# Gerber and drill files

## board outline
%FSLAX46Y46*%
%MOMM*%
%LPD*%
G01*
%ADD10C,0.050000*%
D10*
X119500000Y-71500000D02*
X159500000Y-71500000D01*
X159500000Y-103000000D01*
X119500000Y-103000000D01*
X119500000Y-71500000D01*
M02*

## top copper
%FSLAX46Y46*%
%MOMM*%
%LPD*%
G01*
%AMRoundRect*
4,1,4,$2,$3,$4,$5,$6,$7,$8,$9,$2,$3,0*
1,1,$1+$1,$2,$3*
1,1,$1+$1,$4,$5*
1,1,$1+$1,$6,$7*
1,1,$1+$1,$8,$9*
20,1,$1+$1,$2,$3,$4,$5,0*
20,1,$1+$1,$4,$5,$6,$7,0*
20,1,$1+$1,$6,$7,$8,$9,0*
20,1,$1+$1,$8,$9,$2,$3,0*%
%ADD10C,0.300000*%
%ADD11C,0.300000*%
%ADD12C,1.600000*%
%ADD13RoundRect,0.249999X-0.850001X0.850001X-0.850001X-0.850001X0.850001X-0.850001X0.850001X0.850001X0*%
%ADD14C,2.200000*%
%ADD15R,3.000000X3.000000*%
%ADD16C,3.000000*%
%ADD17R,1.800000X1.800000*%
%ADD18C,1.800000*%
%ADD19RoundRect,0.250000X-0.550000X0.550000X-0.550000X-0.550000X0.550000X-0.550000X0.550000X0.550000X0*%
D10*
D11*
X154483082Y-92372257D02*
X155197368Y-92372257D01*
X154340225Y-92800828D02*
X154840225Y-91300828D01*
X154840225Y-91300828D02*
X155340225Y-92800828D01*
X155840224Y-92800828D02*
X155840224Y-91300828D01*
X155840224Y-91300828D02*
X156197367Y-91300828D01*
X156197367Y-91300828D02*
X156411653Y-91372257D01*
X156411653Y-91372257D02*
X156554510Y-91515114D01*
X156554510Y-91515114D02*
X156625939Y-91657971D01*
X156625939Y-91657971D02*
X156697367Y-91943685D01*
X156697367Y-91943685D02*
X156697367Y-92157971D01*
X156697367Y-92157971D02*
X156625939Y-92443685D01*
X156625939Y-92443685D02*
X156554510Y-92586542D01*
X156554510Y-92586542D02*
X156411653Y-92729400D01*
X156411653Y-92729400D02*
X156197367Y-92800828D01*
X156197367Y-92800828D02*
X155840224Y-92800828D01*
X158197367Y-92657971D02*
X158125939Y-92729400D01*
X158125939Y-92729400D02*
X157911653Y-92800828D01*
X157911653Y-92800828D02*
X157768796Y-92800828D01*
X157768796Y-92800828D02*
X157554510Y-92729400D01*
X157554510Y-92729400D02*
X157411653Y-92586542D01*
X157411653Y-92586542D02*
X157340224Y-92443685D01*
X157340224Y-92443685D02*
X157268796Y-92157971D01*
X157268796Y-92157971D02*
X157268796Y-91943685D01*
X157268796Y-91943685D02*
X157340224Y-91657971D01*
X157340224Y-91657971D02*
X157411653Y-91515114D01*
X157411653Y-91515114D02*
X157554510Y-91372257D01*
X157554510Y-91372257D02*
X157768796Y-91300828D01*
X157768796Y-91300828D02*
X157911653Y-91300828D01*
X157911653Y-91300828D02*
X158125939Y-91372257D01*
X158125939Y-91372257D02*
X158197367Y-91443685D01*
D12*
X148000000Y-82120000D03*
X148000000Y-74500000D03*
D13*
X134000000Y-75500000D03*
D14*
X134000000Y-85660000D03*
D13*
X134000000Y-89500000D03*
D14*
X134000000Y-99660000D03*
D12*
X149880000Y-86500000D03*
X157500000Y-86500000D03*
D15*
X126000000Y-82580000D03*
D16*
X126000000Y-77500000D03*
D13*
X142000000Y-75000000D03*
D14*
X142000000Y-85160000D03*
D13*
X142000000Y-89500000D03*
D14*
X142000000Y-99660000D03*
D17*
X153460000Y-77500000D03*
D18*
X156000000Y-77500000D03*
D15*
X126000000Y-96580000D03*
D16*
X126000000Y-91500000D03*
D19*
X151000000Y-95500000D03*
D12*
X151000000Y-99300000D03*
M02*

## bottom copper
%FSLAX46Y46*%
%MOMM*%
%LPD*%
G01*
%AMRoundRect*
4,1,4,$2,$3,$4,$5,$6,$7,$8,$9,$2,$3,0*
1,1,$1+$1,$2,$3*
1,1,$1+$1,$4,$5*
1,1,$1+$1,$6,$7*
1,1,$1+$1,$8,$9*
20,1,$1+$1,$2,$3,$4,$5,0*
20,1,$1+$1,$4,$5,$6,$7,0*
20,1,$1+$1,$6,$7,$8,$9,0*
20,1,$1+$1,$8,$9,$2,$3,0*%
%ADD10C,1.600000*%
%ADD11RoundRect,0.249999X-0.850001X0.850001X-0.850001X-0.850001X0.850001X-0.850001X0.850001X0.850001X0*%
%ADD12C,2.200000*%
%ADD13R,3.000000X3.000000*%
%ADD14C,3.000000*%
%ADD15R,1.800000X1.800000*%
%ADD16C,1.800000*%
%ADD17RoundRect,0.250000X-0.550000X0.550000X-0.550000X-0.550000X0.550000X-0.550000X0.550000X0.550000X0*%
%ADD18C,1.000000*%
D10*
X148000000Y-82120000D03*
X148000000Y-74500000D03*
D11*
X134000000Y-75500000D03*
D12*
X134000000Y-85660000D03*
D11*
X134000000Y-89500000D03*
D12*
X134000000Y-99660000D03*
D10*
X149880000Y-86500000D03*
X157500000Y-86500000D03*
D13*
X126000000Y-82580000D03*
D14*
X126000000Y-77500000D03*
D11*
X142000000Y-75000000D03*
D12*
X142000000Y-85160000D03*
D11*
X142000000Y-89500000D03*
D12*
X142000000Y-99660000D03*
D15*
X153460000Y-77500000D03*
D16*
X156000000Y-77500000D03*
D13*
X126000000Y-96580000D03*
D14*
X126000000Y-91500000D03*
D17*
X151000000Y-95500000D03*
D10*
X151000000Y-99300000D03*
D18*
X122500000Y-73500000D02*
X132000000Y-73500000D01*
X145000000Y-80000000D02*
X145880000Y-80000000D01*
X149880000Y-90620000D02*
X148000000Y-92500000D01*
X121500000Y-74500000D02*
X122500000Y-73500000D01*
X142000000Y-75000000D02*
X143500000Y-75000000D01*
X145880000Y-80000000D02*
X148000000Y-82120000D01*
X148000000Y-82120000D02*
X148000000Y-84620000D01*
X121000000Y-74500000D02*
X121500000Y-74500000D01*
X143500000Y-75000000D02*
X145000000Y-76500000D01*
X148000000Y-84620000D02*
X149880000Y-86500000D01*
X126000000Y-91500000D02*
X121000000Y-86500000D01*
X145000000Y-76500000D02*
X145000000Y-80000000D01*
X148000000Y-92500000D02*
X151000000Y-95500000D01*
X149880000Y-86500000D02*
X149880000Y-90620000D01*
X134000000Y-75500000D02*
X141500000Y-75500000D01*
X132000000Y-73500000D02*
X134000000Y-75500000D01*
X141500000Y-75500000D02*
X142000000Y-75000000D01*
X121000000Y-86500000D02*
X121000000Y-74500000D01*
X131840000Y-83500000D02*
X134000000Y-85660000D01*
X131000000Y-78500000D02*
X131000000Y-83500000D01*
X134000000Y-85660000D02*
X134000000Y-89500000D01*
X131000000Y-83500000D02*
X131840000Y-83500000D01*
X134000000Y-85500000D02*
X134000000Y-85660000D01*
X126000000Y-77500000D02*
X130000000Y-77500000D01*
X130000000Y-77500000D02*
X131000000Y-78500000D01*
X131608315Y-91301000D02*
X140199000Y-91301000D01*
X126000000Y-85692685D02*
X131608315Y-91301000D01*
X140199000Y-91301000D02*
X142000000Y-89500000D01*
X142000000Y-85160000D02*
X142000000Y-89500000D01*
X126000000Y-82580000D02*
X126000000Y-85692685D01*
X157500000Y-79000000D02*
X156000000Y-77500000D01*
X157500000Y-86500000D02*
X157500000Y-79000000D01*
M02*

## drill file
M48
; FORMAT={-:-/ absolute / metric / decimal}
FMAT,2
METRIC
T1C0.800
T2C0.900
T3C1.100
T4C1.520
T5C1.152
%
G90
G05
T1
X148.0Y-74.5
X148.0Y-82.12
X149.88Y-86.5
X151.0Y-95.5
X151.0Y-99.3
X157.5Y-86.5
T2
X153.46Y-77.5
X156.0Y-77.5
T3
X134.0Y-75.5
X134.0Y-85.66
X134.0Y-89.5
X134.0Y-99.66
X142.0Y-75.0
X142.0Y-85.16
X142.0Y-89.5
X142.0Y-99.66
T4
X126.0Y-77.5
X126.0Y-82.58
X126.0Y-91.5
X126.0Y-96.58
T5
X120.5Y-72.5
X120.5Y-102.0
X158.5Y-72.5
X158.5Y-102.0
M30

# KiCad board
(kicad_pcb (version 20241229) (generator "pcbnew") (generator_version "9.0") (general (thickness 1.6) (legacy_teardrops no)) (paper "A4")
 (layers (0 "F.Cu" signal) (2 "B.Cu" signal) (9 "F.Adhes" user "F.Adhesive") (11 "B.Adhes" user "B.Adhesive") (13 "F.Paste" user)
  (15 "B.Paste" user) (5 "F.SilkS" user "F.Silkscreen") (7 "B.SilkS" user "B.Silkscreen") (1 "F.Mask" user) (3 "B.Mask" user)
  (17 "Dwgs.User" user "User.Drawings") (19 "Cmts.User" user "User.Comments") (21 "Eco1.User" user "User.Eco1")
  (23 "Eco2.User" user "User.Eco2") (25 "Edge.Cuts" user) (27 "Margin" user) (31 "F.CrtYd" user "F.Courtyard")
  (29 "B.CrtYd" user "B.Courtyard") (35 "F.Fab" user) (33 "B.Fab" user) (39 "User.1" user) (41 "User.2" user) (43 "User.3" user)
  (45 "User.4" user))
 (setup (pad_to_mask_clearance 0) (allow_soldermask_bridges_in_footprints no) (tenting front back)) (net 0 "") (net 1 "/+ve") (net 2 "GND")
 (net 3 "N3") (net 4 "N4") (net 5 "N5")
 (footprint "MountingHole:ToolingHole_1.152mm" (layer "F.Cu") (at 158.5 72.5)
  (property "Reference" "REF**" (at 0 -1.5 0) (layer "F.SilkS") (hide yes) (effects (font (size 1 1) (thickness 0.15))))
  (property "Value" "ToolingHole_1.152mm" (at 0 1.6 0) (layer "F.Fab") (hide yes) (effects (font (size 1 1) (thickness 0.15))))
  (pad "" np_thru_hole circle (at 0 0) (size 1.152 1.152) (drill 1.152) (layers "*.Cu" "*.Mask") (solder_mask_margin 0.074))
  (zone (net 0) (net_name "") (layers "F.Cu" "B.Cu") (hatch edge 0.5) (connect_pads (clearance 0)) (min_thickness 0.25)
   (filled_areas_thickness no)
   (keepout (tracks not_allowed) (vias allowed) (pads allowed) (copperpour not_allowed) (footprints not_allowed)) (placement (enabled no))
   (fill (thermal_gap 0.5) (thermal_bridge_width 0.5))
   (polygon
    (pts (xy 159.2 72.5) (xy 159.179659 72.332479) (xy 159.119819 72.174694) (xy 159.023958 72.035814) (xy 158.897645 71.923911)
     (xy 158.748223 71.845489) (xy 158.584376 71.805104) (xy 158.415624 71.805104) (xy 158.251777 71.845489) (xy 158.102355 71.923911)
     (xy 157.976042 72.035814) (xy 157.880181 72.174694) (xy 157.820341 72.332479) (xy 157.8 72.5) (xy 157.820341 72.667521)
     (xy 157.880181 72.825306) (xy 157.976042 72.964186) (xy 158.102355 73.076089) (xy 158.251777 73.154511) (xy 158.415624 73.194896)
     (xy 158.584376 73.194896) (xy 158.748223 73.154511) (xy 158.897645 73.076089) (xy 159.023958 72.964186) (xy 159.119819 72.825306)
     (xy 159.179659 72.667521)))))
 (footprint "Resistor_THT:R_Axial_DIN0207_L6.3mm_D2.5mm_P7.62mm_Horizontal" (layer "F.Cu") (at 148 82.12 90)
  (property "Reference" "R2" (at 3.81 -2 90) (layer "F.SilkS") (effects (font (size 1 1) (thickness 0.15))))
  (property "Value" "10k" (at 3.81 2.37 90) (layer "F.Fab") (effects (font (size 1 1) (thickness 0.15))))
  (pad "1" thru_hole circle (at 0 0 90) (size 1.6 1.6) (drill 0.8) (layers "*.Cu" "*.Mask") (remove_unused_layers no) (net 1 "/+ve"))
  (pad "2" thru_hole circle (at 7.62 0 90) (size 1.6 1.6) (drill 0.8) (layers "*.Cu" "*.Mask") (remove_unused_layers no) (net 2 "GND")))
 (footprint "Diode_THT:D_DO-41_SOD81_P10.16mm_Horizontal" (layer "F.Cu") (at 134 75.5 -90)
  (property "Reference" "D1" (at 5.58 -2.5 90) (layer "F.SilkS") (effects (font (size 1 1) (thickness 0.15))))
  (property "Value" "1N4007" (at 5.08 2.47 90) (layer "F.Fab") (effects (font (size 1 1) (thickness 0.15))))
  (pad "1" thru_hole roundrect (at 0 0 270) (size 2.2 2.2) (drill 1.1) (layers "*.Cu" "*.Mask") (remove_unused_layers no)
   (roundrect_rratio 0.113636) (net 1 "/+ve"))
  (pad "2" thru_hole circle (at 10.16 0 270) (size 2.2 2.2) (drill 1.1) (layers "*.Cu" "*.Mask") (remove_unused_layers no) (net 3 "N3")))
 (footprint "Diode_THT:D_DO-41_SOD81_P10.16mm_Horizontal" (layer "F.Cu") (at 134 89.5 -90)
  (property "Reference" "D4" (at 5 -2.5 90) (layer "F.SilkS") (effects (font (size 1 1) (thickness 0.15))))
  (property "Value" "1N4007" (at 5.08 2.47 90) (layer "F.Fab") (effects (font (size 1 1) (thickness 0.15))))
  (pad "1" thru_hole roundrect (at 0 0 270) (size 2.2 2.2) (drill 1.1) (layers "*.Cu" "*.Mask") (remove_unused_layers no)
   (roundrect_rratio 0.113636) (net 3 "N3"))
  (pad "2" thru_hole circle (at 10.16 0 270) (size 2.2 2.2) (drill 1.1) (layers "*.Cu" "*.Mask") (remove_unused_layers no) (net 2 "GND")))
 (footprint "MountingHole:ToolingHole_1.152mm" (layer "F.Cu") (at 120.5 72.5)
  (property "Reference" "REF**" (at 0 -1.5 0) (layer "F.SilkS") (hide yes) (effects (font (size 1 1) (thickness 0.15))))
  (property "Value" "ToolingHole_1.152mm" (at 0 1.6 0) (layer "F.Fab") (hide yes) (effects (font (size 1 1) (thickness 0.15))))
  (pad "" np_thru_hole circle (at 0 0) (size 1.152 1.152) (drill 1.152) (layers "*.Cu" "*.Mask") (solder_mask_margin 0.074))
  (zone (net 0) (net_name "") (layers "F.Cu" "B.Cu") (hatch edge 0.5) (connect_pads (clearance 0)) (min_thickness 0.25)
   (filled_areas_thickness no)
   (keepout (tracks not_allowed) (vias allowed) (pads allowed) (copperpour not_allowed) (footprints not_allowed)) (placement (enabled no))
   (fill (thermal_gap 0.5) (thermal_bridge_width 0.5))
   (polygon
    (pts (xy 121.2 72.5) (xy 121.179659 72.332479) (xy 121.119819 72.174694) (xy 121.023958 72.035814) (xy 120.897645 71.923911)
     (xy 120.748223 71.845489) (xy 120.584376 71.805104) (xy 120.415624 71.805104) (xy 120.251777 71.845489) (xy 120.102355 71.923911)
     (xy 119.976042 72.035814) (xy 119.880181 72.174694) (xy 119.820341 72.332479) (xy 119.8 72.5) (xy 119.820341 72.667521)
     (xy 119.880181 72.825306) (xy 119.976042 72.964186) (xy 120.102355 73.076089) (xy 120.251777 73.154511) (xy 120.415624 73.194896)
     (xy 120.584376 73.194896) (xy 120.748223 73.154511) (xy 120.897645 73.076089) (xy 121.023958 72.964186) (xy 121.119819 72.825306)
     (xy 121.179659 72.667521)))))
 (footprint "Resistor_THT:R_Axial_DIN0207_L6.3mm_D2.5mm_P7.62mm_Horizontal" (layer "F.Cu") (at 149.88 86.5)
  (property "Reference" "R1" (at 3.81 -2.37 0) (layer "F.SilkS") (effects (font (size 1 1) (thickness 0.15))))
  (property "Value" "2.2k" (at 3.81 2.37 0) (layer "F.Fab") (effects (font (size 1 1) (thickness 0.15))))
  (pad "1" thru_hole circle (at 0 0) (size 1.6 1.6) (drill 0.8) (layers "*.Cu" "*.Mask") (remove_unused_layers no) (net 1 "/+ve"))
  (pad "2" thru_hole circle (at 7.62 0) (size 1.6 1.6) (drill 0.8) (layers "*.Cu" "*.Mask") (remove_unused_layers no) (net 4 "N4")))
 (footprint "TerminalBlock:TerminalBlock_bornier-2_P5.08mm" (layer "F.Cu") (at 126 82.58 90)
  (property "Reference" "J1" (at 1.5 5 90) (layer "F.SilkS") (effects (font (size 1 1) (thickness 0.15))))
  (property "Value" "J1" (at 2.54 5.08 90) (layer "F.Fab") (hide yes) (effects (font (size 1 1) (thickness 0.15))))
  (pad "1" thru_hole rect (at 0 0 90) (size 3 3) (drill 1.52) (layers "*.Cu" "*.Mask") (remove_unused_layers no) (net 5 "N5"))
  (pad "2" thru_hole circle (at 5.08 0 90) (size 3 3) (drill 1.52) (layers "*.Cu" "*.Mask") (remove_unused_layers no) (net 3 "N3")))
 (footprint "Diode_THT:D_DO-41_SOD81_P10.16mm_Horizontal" (layer "F.Cu") (at 142 75 -90)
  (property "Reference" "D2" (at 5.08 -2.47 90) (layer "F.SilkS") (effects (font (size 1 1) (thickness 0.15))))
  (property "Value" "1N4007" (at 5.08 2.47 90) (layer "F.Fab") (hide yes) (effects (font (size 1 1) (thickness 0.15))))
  (pad "1" thru_hole roundrect (at 0 0 270) (size 2.2 2.2) (drill 1.1) (layers "*.Cu" "*.Mask") (remove_unused_layers no)
   (roundrect_rratio 0.113636) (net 1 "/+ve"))
  (pad "2" thru_hole circle (at 10.16 0 270) (size 2.2 2.2) (drill 1.1) (layers "*.Cu" "*.Mask") (remove_unused_layers no) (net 5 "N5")))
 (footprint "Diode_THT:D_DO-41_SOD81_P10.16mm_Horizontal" (layer "F.Cu") (at 142 89.5 -90)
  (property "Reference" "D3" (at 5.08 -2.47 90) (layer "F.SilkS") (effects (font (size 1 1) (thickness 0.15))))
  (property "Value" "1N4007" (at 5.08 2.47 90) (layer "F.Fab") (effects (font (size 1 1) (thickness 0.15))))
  (pad "1" thru_hole roundrect (at 0 0 270) (size 2.2 2.2) (drill 1.1) (layers "*.Cu" "*.Mask") (remove_unused_layers no)
   (roundrect_rratio 0.113636) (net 5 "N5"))
  (pad "2" thru_hole circle (at 10.16 0 270) (size 2.2 2.2) (drill 1.1) (layers "*.Cu" "*.Mask") (remove_unused_layers no) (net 2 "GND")))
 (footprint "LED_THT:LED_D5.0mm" (layer "F.Cu") (at 153.46 77.5)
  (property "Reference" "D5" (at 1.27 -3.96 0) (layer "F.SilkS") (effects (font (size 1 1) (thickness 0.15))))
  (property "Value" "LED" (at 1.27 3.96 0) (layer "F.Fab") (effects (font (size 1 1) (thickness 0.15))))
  (pad "1" thru_hole rect (at 0 0) (size 1.8 1.8) (drill 0.9) (layers "*.Cu" "*.Mask") (remove_unused_layers no) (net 2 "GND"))
  (pad "2" thru_hole circle (at 2.54 0) (size 1.8 1.8) (drill 0.9) (layers "*.Cu" "*.Mask") (remove_unused_layers no) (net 4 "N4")))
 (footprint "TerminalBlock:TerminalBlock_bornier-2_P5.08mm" (layer "F.Cu") (at 126 96.58 90)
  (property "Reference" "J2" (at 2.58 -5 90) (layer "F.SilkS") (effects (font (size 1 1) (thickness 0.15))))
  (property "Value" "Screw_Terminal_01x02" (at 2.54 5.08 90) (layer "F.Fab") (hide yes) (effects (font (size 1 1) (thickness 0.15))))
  (pad "1" thru_hole rect (at 0 0 90) (size 3 3) (drill 1.52) (layers "*.Cu" "*.Mask") (remove_unused_layers no) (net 2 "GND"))
  (pad "2" thru_hole circle (at 5.08 0 90) (size 3 3) (drill 1.52) (layers "*.Cu" "*.Mask") (remove_unused_layers no) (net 1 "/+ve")))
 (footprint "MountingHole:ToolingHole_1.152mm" (layer "F.Cu") (at 158.5 102)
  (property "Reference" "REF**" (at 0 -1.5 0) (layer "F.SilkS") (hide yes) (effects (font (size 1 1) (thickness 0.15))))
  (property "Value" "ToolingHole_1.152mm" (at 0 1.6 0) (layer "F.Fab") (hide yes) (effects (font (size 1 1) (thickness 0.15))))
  (pad "" np_thru_hole circle (at 0 0) (size 1.152 1.152) (drill 1.152) (layers "*.Cu" "*.Mask") (solder_mask_margin 0.074))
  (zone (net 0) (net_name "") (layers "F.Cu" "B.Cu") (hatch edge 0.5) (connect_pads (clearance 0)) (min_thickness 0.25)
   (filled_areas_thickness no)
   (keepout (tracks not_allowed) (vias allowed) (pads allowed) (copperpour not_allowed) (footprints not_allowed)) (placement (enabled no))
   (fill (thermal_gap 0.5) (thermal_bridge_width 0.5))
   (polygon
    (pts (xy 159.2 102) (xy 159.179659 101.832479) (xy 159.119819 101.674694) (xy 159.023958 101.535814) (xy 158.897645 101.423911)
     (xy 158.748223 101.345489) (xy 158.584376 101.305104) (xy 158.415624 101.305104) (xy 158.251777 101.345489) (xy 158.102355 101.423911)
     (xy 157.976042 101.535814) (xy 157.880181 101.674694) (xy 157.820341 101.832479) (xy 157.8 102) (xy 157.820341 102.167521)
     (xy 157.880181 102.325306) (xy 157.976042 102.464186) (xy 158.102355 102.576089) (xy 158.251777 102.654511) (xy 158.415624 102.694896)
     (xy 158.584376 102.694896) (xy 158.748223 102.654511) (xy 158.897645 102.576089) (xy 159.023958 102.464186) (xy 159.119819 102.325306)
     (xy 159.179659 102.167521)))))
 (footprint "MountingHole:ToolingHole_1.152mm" (layer "F.Cu") (at 120.5 102)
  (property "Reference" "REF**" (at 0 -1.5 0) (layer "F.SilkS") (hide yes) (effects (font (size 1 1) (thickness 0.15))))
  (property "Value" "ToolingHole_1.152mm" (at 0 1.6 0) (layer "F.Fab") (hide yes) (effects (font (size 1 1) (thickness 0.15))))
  (pad "" np_thru_hole circle (at 0 0) (size 1.152 1.152) (drill 1.152) (layers "*.Cu" "*.Mask") (solder_mask_margin 0.074))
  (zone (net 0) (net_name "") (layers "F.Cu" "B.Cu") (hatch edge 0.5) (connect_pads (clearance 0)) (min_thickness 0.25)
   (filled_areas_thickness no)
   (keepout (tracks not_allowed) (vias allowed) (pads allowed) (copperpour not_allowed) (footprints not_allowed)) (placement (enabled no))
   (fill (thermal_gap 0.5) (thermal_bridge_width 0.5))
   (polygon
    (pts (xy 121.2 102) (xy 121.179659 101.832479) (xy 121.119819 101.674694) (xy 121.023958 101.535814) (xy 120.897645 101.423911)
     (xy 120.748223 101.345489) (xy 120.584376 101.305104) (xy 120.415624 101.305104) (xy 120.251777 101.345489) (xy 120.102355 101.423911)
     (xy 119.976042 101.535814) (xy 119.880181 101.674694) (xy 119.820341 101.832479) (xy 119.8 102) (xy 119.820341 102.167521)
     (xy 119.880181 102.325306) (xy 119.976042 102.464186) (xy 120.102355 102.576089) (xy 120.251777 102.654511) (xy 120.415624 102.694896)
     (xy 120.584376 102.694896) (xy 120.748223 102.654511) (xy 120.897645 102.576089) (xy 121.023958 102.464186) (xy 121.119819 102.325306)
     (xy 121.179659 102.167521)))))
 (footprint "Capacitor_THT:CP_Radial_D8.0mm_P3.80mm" (layer "F.Cu") (at 151 95.5 -90)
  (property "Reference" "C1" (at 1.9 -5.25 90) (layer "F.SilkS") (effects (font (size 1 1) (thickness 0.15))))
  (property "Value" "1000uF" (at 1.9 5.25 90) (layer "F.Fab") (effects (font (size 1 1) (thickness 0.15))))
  (pad "1" thru_hole roundrect (at 0 0 270) (size 1.6 1.6) (drill 0.8) (layers "*.Cu" "*.Mask") (remove_unused_layers no)
   (roundrect_rratio 0.15625) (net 1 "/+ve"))
  (pad "2" thru_hole circle (at 3.8 0 270) (size 1.6 1.6) (drill 0.8) (layers "*.Cu" "*.Mask") (remove_unused_layers no) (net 2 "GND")))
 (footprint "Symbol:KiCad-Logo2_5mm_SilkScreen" (layer "B.Cu") (at 137 99.5 180)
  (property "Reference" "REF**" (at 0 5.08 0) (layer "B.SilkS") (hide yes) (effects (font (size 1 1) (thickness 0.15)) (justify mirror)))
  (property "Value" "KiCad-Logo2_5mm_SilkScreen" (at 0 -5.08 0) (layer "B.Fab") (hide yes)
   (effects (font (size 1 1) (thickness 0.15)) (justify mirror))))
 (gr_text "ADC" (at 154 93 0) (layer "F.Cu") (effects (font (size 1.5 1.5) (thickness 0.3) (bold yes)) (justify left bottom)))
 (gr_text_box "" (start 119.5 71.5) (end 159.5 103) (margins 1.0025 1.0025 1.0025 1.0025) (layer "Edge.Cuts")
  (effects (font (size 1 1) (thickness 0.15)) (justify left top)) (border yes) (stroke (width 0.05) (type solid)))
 (segment (start 122.5 73.5) (end 132 73.5) (width 1) (layer "B.Cu") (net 1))
 (segment (start 145 80) (end 145.88 80) (width 1) (layer "B.Cu") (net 1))
 (segment (start 149.88 90.62) (end 148 92.5) (width 1) (layer "B.Cu") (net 1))
 (segment (start 121.5 74.5) (end 122.5 73.5) (width 1) (layer "B.Cu") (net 1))
 (segment (start 142 75) (end 143.5 75) (width 1) (layer "B.Cu") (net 1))
 (segment (start 145.88 80) (end 148 82.12) (width 1) (layer "B.Cu") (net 1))
 (segment (start 148 82.12) (end 148 84.62) (width 1) (layer "B.Cu") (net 1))
 (segment (start 121 74.5) (end 121.5 74.5) (width 1) (layer "B.Cu") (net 1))
 (segment (start 143.5 75) (end 145 76.5) (width 1) (layer "B.Cu") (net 1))
 (segment (start 148 84.62) (end 149.88 86.5) (width 1) (layer "B.Cu") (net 1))
 (segment (start 126 91.5) (end 121 86.5) (width 1) (layer "B.Cu") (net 1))
 (segment (start 145 76.5) (end 145 80) (width 1) (layer "B.Cu") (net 1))
 (segment (start 148 92.5) (end 151 95.5) (width 1) (layer "B.Cu") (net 1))
 (segment (start 149.88 86.5) (end 149.88 90.62) (width 1) (layer "B.Cu") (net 1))
 (segment (start 134 75.5) (end 141.5 75.5) (width 1) (layer "B.Cu") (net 1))
 (segment (start 132 73.5) (end 134 75.5) (width 1) (layer "B.Cu") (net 1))
 (segment (start 141.5 75.5) (end 142 75) (width 1) (layer "B.Cu") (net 1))
 (segment (start 121 86.5) (end 121 74.5) (width 1) (layer "B.Cu") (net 1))
 (segment (start 131.84 83.5) (end 134 85.66) (width 1) (layer "B.Cu") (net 3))
 (segment (start 131 78.5) (end 131 83.5) (width 1) (layer "B.Cu") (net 3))
 (segment (start 134 85.66) (end 134 89.5) (width 1) (layer "B.Cu") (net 3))
 (segment (start 131 83.5) (end 131.84 83.5) (width 1) (layer "B.Cu") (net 3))
 (segment (start 134 85.5) (end 134 85.66) (width 1) (layer "B.Cu") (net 3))
 (segment (start 126 77.5) (end 130 77.5) (width 1) (layer "B.Cu") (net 3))
 (segment (start 130 77.5) (end 131 78.5) (width 1) (layer "B.Cu") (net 3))
 (segment (start 131.608315 91.301) (end 140.199 91.301) (width 1) (layer "B.Cu") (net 5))
 (segment (start 126 85.692685) (end 131.608315 91.301) (width 1) (layer "B.Cu") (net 5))
 (segment (start 140.199 91.301) (end 142 89.5) (width 1) (layer "B.Cu") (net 5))
 (segment (start 142 85.16) (end 142 89.5) (width 1) (layer "B.Cu") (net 5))
 (segment (start 126 82.58) (end 126 85.692685) (width 1) (layer "B.Cu") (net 5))
 (segment (start 157.5 79) (end 156 77.5) (width 1) (layer "B.Cu") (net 4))
 (segment (start 157.5 86.5) (end 157.5 79) (width 1) (layer "B.Cu") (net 4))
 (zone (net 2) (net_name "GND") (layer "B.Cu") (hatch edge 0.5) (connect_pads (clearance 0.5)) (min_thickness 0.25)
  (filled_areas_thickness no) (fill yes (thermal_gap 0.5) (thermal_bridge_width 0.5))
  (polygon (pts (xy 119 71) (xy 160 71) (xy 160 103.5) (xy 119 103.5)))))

